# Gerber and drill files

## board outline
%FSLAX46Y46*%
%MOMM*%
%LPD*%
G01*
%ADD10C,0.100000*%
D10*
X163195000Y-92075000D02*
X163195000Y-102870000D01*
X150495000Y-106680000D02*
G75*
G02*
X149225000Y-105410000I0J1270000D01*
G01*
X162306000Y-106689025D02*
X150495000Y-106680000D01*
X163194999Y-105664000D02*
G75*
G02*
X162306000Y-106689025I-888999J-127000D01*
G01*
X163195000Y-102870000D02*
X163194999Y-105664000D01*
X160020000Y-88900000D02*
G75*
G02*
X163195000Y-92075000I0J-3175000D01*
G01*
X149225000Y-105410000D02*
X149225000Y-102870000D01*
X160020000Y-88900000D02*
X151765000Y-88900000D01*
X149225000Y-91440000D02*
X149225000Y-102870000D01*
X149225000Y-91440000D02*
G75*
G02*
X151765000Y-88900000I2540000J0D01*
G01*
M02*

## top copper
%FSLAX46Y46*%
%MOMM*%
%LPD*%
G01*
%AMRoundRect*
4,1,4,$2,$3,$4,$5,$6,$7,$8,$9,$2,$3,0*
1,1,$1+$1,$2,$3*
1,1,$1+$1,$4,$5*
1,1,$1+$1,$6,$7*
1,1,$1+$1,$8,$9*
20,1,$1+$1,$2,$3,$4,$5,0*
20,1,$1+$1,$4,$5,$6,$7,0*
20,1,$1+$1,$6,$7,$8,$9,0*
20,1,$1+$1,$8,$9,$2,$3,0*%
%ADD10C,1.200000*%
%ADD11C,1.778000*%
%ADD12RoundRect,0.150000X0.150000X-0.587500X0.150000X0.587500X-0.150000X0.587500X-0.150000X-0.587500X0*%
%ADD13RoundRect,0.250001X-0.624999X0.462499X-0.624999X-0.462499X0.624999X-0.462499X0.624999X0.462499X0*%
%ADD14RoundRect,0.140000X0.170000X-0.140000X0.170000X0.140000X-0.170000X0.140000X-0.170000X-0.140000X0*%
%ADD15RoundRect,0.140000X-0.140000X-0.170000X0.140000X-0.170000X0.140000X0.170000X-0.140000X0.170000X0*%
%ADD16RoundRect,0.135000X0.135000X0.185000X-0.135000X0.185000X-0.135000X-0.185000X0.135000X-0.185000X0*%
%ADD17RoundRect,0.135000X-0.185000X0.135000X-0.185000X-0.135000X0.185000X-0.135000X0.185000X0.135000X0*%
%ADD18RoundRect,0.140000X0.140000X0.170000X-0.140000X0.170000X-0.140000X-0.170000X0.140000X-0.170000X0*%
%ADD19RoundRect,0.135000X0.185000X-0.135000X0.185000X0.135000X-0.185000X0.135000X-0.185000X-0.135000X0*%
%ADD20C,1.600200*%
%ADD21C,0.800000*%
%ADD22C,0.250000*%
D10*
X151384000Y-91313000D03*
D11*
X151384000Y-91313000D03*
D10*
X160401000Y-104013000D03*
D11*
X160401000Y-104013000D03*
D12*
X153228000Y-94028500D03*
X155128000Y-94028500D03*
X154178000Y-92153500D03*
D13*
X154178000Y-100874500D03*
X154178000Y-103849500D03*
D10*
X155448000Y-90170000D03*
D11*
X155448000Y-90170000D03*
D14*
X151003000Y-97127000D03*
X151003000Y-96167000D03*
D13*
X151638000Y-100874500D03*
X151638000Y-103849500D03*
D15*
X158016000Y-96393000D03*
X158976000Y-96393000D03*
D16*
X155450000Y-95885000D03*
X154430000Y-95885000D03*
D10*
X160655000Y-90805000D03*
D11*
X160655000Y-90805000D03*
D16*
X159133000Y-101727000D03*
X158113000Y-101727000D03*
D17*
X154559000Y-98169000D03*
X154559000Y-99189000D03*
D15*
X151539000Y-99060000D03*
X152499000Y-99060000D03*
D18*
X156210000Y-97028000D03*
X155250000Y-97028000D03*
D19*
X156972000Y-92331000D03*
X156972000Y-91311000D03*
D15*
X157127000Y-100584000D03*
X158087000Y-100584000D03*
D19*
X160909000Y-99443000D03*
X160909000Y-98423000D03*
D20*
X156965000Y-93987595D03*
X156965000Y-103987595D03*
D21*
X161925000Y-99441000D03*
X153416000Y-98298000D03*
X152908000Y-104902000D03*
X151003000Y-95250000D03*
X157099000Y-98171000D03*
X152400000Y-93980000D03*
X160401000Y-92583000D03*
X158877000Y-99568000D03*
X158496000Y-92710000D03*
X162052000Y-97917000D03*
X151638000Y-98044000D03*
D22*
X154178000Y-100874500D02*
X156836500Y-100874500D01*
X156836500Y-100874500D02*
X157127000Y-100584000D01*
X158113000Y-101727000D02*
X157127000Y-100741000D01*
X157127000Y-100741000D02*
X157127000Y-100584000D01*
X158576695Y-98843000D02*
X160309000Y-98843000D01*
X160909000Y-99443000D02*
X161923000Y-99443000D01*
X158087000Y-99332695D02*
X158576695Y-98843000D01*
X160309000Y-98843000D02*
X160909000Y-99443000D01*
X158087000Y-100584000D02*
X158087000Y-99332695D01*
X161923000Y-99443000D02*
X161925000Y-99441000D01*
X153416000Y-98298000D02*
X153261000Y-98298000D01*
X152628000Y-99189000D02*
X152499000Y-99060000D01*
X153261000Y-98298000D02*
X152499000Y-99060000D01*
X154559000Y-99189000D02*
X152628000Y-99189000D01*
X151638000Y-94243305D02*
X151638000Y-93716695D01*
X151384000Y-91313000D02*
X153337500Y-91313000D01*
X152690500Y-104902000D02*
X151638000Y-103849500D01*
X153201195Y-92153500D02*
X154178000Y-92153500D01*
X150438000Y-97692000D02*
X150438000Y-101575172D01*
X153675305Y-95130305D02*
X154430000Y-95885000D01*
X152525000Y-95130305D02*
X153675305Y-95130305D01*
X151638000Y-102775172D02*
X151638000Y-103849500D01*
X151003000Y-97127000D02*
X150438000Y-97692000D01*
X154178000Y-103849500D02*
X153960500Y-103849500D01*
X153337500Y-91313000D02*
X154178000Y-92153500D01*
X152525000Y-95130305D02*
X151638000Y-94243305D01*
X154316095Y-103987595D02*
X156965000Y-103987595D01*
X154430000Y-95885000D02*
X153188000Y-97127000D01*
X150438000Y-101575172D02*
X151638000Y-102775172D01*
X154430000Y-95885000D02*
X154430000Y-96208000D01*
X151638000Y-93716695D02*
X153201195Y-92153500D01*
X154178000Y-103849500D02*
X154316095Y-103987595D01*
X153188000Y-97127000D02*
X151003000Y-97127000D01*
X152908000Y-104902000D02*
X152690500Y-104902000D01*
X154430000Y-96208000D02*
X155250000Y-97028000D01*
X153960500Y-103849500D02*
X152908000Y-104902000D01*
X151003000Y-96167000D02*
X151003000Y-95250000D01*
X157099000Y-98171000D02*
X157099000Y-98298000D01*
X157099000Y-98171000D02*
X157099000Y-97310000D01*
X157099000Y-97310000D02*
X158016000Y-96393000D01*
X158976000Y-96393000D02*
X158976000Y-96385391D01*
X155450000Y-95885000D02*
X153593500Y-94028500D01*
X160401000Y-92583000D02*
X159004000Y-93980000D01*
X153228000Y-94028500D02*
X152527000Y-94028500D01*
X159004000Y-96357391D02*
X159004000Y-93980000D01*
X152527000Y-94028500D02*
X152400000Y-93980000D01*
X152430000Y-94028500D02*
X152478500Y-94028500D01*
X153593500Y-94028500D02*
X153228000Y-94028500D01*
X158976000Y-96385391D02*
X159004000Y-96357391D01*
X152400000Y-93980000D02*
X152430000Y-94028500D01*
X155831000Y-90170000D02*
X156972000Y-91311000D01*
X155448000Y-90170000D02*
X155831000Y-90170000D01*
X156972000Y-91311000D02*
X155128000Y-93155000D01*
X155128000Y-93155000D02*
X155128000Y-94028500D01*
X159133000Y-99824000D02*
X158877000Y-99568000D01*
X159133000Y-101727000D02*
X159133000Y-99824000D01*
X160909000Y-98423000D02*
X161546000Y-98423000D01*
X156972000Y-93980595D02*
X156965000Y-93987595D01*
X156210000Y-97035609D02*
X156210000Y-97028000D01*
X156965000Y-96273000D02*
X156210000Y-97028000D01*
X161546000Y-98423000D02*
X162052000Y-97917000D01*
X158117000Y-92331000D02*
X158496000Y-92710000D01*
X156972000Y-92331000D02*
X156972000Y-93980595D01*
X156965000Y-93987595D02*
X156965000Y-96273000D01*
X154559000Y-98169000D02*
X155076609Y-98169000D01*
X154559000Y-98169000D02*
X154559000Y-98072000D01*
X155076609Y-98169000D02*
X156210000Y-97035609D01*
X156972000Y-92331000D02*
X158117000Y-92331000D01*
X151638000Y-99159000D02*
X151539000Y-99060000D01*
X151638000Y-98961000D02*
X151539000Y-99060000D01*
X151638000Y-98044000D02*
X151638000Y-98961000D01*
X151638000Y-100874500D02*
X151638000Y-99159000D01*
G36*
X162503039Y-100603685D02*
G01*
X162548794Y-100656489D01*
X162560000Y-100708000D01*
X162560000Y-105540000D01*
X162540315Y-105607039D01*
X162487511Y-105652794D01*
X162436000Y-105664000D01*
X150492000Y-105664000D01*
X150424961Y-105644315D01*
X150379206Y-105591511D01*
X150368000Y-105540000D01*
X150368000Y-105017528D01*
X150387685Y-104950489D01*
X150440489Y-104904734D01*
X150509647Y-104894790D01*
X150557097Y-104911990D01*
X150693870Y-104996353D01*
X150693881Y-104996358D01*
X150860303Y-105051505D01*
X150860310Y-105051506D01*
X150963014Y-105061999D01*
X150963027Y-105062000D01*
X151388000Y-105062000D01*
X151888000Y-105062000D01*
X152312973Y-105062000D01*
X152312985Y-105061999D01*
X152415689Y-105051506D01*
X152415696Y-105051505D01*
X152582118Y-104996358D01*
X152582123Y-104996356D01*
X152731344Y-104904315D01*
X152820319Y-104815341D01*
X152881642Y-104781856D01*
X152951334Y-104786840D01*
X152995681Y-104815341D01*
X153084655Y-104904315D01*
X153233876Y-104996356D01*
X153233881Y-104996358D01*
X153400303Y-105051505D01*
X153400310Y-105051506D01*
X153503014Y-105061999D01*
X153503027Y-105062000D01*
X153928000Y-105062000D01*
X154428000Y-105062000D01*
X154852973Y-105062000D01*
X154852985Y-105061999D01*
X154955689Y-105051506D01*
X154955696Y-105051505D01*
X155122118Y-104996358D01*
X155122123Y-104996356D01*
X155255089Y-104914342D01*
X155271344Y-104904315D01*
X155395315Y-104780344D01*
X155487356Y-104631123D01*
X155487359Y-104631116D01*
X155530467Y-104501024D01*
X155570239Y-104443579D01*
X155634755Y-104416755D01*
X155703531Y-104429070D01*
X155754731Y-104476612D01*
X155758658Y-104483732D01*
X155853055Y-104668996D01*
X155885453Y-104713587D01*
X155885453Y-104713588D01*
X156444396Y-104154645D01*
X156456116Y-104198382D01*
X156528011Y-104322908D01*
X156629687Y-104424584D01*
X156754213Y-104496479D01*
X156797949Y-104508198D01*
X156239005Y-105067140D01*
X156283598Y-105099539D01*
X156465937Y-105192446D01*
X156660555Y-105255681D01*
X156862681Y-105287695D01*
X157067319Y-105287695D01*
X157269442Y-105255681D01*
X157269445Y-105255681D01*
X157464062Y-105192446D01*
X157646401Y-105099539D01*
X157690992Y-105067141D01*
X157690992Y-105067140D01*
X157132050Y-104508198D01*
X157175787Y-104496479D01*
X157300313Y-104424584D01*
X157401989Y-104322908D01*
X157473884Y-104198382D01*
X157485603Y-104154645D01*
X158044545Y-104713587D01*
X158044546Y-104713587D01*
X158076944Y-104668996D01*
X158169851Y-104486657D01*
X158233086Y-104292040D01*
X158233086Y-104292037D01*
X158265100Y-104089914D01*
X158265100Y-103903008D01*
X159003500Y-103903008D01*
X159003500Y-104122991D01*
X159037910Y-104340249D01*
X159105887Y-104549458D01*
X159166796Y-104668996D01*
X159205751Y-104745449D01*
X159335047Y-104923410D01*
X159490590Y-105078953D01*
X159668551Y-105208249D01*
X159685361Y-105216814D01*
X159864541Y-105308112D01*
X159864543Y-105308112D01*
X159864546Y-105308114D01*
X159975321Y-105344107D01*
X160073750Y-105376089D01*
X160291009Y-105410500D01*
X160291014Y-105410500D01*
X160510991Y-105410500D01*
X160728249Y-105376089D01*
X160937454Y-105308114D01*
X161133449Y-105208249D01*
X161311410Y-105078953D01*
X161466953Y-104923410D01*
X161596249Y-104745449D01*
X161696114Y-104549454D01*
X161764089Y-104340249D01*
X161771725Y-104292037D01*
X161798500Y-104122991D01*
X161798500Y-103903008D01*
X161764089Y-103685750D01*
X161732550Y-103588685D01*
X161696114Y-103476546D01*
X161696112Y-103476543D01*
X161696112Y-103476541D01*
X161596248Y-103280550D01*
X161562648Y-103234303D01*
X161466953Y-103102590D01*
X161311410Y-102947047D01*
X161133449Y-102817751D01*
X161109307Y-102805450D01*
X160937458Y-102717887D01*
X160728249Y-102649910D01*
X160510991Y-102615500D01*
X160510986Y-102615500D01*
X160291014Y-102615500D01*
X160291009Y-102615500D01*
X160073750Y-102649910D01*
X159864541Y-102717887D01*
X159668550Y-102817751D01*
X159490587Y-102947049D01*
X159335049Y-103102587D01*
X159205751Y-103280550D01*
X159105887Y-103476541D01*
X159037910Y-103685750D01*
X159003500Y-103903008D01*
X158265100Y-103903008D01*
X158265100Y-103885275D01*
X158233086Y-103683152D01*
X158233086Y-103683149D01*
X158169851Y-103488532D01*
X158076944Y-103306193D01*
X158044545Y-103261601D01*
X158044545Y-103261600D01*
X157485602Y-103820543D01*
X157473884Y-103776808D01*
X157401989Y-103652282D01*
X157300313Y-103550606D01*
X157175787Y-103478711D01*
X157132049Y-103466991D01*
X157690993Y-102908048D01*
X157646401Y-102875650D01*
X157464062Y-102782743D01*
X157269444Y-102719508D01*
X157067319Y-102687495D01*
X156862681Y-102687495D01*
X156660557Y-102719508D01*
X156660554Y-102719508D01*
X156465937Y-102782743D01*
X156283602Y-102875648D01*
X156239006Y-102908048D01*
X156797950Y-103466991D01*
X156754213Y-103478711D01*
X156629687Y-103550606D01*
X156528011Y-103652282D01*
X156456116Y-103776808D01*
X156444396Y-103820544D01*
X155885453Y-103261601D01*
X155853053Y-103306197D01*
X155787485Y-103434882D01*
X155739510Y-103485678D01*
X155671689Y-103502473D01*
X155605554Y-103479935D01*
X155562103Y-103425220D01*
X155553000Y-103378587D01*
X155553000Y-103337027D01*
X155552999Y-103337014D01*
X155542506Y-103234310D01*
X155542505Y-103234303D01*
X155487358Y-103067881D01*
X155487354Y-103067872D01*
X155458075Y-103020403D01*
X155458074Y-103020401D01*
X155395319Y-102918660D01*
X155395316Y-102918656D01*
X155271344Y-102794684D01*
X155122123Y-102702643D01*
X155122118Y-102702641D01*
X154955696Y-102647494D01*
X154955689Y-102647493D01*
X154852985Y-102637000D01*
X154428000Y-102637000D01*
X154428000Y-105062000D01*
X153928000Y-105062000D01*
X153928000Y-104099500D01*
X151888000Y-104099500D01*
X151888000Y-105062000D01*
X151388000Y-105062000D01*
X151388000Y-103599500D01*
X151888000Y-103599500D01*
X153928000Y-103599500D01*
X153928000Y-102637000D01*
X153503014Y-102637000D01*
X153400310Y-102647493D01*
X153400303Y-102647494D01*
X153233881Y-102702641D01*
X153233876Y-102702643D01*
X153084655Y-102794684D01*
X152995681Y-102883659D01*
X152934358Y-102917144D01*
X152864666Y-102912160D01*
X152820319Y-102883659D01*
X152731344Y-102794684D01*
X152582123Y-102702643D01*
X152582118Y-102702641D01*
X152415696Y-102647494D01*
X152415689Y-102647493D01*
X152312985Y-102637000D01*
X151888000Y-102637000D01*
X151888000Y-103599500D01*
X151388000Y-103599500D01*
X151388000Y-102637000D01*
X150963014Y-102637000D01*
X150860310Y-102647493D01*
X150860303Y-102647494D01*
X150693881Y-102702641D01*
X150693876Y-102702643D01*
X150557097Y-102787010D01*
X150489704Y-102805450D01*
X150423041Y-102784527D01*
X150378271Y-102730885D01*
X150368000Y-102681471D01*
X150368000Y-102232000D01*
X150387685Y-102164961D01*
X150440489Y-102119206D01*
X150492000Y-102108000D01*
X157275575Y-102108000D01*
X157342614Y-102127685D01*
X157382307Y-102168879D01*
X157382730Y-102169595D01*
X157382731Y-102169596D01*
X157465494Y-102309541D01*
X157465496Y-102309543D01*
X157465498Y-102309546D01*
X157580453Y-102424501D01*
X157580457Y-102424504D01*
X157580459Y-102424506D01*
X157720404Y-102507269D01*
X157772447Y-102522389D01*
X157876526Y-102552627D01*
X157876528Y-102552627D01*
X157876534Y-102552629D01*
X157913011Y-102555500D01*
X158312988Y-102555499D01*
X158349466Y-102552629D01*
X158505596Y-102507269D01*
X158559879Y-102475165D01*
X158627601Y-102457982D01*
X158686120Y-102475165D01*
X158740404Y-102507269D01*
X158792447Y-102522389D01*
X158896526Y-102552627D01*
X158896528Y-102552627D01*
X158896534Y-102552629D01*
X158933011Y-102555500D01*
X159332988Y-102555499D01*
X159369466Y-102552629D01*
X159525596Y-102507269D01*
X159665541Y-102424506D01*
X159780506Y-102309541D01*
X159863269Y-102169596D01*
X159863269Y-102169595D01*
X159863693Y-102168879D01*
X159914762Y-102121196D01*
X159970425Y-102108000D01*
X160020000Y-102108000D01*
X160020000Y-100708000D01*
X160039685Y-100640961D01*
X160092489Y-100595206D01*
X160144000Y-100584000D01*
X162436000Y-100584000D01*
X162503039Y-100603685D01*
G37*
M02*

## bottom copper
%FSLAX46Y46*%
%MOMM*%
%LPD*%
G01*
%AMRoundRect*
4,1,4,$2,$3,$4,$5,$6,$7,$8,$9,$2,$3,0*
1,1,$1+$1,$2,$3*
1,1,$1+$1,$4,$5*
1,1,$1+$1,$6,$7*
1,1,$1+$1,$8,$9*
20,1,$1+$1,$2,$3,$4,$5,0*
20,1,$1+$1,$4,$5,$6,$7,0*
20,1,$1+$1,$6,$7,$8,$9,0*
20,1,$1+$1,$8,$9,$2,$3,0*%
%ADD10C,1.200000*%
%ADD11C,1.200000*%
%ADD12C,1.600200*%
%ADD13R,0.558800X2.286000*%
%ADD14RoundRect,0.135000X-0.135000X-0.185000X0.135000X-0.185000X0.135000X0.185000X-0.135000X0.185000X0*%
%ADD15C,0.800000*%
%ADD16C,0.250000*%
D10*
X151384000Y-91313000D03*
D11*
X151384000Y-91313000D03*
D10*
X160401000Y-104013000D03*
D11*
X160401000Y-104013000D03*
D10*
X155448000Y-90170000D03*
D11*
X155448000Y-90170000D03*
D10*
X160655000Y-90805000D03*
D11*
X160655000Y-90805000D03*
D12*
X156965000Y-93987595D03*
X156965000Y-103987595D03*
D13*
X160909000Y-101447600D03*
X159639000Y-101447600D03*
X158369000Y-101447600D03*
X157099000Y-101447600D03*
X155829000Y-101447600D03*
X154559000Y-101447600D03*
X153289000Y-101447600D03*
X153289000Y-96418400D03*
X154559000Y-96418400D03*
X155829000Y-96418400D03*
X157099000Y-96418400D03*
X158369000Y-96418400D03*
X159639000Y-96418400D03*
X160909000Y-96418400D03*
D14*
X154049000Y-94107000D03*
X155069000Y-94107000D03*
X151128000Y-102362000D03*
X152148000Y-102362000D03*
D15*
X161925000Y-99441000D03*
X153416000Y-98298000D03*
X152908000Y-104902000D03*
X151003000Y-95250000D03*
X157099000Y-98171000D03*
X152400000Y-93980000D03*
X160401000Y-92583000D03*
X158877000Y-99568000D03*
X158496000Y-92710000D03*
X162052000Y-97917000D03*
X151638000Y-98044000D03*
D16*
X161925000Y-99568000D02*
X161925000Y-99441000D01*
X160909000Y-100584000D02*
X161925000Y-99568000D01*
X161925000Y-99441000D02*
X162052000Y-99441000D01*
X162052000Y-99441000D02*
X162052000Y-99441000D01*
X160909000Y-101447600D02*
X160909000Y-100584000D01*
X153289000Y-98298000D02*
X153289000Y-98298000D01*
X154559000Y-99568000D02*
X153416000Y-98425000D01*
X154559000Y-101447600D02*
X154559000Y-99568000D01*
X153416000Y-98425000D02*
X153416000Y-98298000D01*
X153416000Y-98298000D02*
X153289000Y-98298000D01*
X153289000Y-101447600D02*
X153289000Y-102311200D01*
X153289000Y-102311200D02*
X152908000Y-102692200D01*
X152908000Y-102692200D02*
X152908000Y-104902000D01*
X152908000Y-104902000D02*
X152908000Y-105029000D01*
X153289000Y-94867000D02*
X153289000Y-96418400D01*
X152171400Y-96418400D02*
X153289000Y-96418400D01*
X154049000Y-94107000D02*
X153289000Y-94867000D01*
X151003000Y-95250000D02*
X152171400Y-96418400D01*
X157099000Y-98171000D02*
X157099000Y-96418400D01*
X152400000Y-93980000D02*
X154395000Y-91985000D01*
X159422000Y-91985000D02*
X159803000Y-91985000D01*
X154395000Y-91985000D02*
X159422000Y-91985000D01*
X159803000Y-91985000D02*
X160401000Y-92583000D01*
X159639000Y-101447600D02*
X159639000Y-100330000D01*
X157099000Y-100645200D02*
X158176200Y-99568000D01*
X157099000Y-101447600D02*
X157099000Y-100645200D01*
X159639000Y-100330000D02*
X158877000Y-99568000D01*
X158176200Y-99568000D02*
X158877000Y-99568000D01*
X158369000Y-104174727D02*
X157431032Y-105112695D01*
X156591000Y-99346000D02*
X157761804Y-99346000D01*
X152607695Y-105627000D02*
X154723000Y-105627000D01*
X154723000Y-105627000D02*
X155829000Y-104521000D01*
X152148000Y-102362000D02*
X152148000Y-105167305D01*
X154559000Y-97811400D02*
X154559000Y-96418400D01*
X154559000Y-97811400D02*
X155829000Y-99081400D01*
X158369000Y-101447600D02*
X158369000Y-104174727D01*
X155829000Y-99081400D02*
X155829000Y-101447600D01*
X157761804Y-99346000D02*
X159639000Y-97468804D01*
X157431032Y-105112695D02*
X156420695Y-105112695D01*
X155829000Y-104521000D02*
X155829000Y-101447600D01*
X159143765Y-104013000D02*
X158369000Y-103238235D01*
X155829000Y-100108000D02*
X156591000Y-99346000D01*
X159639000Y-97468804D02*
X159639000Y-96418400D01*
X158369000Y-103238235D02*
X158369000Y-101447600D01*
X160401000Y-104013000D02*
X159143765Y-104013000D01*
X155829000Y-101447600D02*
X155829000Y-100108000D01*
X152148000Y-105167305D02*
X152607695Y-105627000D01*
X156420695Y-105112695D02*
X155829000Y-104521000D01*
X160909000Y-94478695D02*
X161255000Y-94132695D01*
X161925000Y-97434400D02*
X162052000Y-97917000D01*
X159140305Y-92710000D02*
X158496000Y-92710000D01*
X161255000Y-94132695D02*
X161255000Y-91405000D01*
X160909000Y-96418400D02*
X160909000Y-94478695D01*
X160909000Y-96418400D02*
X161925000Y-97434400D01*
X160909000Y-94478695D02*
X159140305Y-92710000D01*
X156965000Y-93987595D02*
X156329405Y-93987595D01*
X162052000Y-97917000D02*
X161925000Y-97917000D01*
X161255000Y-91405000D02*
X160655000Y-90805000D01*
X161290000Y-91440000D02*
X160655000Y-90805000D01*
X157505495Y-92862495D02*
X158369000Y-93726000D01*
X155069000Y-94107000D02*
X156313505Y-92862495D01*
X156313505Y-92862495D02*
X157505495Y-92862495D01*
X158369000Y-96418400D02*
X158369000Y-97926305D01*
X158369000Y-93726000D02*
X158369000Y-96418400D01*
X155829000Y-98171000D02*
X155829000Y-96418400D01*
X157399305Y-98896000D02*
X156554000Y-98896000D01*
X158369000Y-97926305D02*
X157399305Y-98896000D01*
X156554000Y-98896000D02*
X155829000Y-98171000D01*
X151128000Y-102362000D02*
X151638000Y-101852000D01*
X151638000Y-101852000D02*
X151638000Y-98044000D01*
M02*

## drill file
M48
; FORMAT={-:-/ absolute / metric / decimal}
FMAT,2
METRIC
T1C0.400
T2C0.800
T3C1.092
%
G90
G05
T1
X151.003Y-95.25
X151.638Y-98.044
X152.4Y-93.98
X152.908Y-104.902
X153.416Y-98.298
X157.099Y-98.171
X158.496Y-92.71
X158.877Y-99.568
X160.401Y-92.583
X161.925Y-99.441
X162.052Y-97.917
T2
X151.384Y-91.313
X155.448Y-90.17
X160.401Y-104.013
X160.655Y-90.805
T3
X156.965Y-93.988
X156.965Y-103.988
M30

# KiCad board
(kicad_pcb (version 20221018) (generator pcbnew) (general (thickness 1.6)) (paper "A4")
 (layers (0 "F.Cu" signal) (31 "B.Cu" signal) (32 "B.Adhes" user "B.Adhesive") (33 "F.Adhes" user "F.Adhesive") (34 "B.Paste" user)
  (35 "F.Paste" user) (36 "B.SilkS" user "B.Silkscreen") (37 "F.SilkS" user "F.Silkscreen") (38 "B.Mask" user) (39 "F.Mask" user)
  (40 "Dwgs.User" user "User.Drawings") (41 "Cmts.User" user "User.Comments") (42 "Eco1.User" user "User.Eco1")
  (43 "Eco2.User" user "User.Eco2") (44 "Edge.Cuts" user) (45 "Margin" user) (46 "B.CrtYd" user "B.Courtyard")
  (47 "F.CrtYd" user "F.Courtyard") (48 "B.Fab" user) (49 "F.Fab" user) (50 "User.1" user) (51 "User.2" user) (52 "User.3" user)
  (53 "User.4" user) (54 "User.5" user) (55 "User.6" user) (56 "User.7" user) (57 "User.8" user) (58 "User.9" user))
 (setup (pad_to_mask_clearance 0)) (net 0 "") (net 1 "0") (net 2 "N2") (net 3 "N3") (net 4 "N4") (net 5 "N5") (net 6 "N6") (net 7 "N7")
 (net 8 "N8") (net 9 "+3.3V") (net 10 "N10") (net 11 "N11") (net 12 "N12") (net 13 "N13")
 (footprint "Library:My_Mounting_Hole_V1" (layer "F.Cu") (at 151.384 91.313)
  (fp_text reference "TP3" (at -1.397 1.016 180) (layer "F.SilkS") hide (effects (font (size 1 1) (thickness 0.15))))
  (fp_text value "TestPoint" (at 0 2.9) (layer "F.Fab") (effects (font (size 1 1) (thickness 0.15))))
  (pad "1" thru_hole circle (at 0 0) (size 1.2 1.2) (drill 0.8) (layers "*.Cu" "*.Mask") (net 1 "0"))
  (pad "1" connect circle (at 0 0) (size 1.2 1.2) (layers "B.Cu" "B.Mask") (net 1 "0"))
  (pad "1" connect circle (at 0 0) (size 1.778 1.778) (layers "F.Cu" "F.Mask") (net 1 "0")))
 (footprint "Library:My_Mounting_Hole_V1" (layer "F.Cu") (at 160.401 104.013)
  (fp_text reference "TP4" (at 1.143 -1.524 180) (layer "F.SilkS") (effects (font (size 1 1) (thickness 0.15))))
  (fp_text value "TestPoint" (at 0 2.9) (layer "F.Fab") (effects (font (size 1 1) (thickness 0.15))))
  (pad "1" thru_hole circle (at 0 0) (size 1.2 1.2) (drill 0.8) (layers "*.Cu" "*.Mask") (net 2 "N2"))
  (pad "1" connect circle (at 0 0) (size 1.2 1.2) (layers "B.Cu" "B.Mask") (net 2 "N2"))
  (pad "1" connect circle (at 0 0) (size 1.778 1.778) (layers "F.Cu" "F.Mask") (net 2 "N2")))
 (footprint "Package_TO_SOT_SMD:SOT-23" (layer "F.Cu") (at 154.178 93.091 90)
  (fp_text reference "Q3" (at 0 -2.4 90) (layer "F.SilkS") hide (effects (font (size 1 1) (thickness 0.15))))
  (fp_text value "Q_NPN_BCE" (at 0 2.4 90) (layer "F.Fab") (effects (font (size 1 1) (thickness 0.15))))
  (pad "1" smd roundrect (at -0.9375 -0.95 90) (size 1.475 0.6) (layers "F.Cu" "F.Paste" "F.Mask") (roundrect_rratio 0.25) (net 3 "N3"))
  (pad "2" smd roundrect (at -0.9375 0.95 90) (size 1.475 0.6) (layers "F.Cu" "F.Paste" "F.Mask") (roundrect_rratio 0.25) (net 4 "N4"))
  (pad "3" smd roundrect (at 0.9375 0 90) (size 1.475 0.6) (layers "F.Cu" "F.Paste" "F.Mask") (roundrect_rratio 0.25) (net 1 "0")))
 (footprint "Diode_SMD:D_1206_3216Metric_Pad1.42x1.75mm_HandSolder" (layer "F.Cu") (at 154.178 102.362 -90)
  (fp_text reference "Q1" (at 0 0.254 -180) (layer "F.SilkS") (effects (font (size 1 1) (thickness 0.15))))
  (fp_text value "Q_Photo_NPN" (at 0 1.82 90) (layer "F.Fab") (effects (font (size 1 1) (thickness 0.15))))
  (pad "1" smd roundrect (at -1.4875 0 270) (size 1.425 1.75) (layers "F.Cu" "F.Paste" "F.Mask") (roundrect_rratio 0.1754392982)
   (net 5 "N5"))
  (pad "2" smd roundrect (at 1.4875 0 270) (size 1.425 1.75) (layers "F.Cu" "F.Paste" "F.Mask") (roundrect_rratio 0.1754392982) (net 1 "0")))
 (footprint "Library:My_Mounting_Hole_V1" (layer "F.Cu") (at 155.448 90.17)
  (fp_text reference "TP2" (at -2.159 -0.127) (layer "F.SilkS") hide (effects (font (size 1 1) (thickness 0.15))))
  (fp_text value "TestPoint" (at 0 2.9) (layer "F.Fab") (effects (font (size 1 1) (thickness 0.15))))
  (pad "1" thru_hole circle (at 0 0) (size 1.2 1.2) (drill 0.8) (layers "*.Cu" "*.Mask") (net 4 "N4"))
  (pad "1" connect circle (at 0 0) (size 1.2 1.2) (layers "B.Cu" "B.Mask") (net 4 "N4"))
  (pad "1" connect circle (at 0 0) (size 1.778 1.778) (layers "F.Cu" "F.Mask") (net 4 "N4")))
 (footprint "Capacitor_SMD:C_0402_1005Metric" (layer "F.Cu") (at 151.003 96.647 90)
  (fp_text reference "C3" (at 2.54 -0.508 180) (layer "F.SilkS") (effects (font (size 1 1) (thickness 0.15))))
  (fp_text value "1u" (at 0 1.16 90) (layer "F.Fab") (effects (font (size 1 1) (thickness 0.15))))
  (pad "1" smd roundrect (at -0.48 0 90) (size 0.56 0.62) (layers "F.Cu" "F.Paste" "F.Mask") (roundrect_rratio 0.25) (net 1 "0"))
  (pad "2" smd roundrect (at 0.48 0 90) (size 0.56 0.62) (layers "F.Cu" "F.Paste" "F.Mask") (roundrect_rratio 0.25) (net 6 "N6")))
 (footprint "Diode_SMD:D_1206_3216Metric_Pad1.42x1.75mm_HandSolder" (layer "F.Cu") (at 151.638 102.362 -90)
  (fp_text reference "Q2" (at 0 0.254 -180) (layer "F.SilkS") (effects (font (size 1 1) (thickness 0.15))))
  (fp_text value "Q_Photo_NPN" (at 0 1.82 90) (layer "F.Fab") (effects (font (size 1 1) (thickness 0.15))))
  (pad "1" smd roundrect (at -1.4875 0 270) (size 1.425 1.75) (layers "F.Cu" "F.Paste" "F.Mask") (roundrect_rratio 0.1754392982)
   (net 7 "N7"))
  (pad "2" smd roundrect (at 1.4875 0 270) (size 1.425 1.75) (layers "F.Cu" "F.Paste" "F.Mask") (roundrect_rratio 0.1754392982) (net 1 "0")))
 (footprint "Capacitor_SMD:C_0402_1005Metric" (layer "F.Cu") (at 158.496 96.393)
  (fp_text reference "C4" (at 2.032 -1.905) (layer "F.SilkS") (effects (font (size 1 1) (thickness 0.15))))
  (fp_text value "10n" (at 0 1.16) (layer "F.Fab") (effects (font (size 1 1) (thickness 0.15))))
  (pad "1" smd roundrect (at -0.48 0) (size 0.56 0.62) (layers "F.Cu" "F.Paste" "F.Mask") (roundrect_rratio 0.25) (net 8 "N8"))
  (pad "2" smd roundrect (at 0.48 0) (size 0.56 0.62) (layers "F.Cu" "F.Paste" "F.Mask") (roundrect_rratio 0.25) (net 3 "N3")))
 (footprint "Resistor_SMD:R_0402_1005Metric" (layer "F.Cu") (at 154.94 95.885 180)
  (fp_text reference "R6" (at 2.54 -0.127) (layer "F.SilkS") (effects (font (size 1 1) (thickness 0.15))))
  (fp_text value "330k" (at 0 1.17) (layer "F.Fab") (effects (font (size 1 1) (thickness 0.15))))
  (pad "1" smd roundrect (at -0.51 0 180) (size 0.54 0.64) (layers "F.Cu" "F.Paste" "F.Mask") (roundrect_rratio 0.25) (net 3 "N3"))
  (pad "2" smd roundrect (at 0.51 0 180) (size 0.54 0.64) (layers "F.Cu" "F.Paste" "F.Mask") (roundrect_rratio 0.25) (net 1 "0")))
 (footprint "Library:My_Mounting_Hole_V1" (layer "F.Cu") (at 160.655 90.805)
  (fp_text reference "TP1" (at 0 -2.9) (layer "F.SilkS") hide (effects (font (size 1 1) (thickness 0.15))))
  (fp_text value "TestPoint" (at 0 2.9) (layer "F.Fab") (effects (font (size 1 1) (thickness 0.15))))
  (pad "1" thru_hole circle (at 0 0) (size 1.2 1.2) (drill 0.8) (layers "*.Cu" "*.Mask") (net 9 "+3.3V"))
  (pad "1" connect circle (at 0 0) (size 1.2 1.2) (layers "B.Cu" "B.Mask") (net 9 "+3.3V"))
  (pad "1" connect circle (at 0 0) (size 1.778 1.778) (layers "F.Cu" "F.Mask") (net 9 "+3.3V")))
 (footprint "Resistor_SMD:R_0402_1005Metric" (layer "F.Cu") (at 158.623 101.727 180)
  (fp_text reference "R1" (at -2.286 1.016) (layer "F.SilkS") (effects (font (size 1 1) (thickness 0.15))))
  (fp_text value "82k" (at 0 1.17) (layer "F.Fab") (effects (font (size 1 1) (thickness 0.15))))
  (pad "1" smd roundrect (at -0.51 0 180) (size 0.54 0.64) (layers "F.Cu" "F.Paste" "F.Mask") (roundrect_rratio 0.25) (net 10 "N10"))
  (pad "2" smd roundrect (at 0.51 0 180) (size 0.54 0.64) (layers "F.Cu" "F.Paste" "F.Mask") (roundrect_rratio 0.25) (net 5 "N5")))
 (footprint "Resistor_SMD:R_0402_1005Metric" (layer "F.Cu") (at 154.559 98.679 -90)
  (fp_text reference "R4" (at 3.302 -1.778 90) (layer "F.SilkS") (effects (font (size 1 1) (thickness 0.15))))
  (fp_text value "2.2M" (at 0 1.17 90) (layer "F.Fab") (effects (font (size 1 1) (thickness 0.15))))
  (pad "1" smd roundrect (at -0.51 0 270) (size 0.54 0.64) (layers "F.Cu" "F.Paste" "F.Mask") (roundrect_rratio 0.25) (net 9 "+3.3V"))
  (pad "2" smd roundrect (at 0.51 0 270) (size 0.54 0.64) (layers "F.Cu" "F.Paste" "F.Mask") (roundrect_rratio 0.25) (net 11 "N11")))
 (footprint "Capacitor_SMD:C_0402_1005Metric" (layer "F.Cu") (at 152.019 99.06)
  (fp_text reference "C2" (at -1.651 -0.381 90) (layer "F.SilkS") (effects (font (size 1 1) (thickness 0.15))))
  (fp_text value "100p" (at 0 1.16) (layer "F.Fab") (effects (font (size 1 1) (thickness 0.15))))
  (pad "1" smd roundrect (at -0.48 0) (size 0.56 0.62) (layers "F.Cu" "F.Paste" "F.Mask") (roundrect_rratio 0.25) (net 7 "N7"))
  (pad "2" smd roundrect (at 0.48 0) (size 0.56 0.62) (layers "F.Cu" "F.Paste" "F.Mask") (roundrect_rratio 0.25) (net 11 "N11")))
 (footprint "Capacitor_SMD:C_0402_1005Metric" (layer "F.Cu") (at 155.73 97.028 180)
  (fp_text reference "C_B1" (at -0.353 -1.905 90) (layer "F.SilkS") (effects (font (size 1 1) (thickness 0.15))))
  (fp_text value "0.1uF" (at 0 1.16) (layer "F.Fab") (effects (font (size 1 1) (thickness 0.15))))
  (pad "1" smd roundrect (at -0.48 0 180) (size 0.56 0.62) (layers "F.Cu" "F.Paste" "F.Mask") (roundrect_rratio 0.25) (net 9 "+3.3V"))
  (pad "2" smd roundrect (at 0.48 0 180) (size 0.56 0.62) (layers "F.Cu" "F.Paste" "F.Mask") (roundrect_rratio 0.25) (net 1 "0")))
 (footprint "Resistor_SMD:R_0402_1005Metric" (layer "F.Cu") (at 156.972 91.821 90)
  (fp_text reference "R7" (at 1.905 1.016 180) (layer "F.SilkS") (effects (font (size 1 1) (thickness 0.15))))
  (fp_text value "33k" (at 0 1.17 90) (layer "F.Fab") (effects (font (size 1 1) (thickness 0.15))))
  (pad "1" smd roundrect (at -0.51 0 90) (size 0.54 0.64) (layers "F.Cu" "F.Paste" "F.Mask") (roundrect_rratio 0.25) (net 9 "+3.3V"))
  (pad "2" smd roundrect (at 0.51 0 90) (size 0.54 0.64) (layers "F.Cu" "F.Paste" "F.Mask") (roundrect_rratio 0.25) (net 4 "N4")))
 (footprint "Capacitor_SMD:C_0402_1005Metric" (layer "F.Cu") (at 157.607 100.584)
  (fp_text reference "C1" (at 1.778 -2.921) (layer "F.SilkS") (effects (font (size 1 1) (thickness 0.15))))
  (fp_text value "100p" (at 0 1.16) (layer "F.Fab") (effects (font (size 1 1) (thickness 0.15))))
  (pad "1" smd roundrect (at -0.48 0) (size 0.56 0.62) (layers "F.Cu" "F.Paste" "F.Mask") (roundrect_rratio 0.25) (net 5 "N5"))
  (pad "2" smd roundrect (at 0.48 0) (size 0.56 0.62) (layers "F.Cu" "F.Paste" "F.Mask") (roundrect_rratio 0.25) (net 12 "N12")))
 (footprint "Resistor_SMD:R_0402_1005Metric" (layer "F.Cu") (at 160.909 98.933 90)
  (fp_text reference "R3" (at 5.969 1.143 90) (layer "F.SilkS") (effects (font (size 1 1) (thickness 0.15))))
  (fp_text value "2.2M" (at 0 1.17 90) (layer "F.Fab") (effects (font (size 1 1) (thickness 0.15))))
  (pad "1" smd roundrect (at -0.51 0 90) (size 0.54 0.64) (layers "F.Cu" "F.Paste" "F.Mask") (roundrect_rratio 0.25) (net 12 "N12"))
  (pad "2" smd roundrect (at 0.51 0 90) (size 0.54 0.64) (layers "F.Cu" "F.Paste" "F.Mask") (roundrect_rratio 0.25) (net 9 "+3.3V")))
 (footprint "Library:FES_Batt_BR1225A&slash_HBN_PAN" (layer "B.Cu") (at 156.965 93.987595 180)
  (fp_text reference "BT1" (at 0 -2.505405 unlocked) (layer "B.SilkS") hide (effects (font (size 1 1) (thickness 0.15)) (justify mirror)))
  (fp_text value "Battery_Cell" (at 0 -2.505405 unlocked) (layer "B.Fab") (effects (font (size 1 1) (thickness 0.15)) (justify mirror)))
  (pad "1" thru_hole circle (at 0 0 180) (size 1.6002 1.6002) (drill 1.0922) (layers "*.Cu" "*.Mask") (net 9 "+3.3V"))
  (pad "2" thru_hole circle (at 0 -10 180) (size 1.6002 1.6002) (drill 1.0922) (layers "*.Cu" "*.Mask") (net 1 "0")))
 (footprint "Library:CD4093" (layer "B.Cu") (at 157.099 98.933 90)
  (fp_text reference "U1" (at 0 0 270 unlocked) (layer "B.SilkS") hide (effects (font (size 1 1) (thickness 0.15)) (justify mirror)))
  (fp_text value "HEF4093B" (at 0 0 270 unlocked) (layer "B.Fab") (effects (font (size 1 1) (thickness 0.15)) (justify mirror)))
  (pad "1" smd rect (at -2.5146 3.81 90) (size 2.286 0.5588) (layers "B.Cu" "B.Paste" "B.Mask") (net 12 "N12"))
  (pad "2" smd rect (at -2.5146 2.54 90) (size 2.286 0.5588) (layers "B.Cu" "B.Paste" "B.Mask") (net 10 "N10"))
  (pad "3" smd rect (at -2.5146 1.27 90) (size 2.286 0.5588) (layers "B.Cu" "B.Paste" "B.Mask") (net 2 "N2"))
  (pad "4" smd rect (at -2.5146 0 90) (size 2.286 0.5588) (layers "B.Cu" "B.Paste" "B.Mask") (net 10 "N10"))
  (pad "5" smd rect (at -2.5146 -1.27 90) (size 2.286 0.5588) (layers "B.Cu" "B.Paste" "B.Mask") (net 2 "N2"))
  (pad "6" smd rect (at -2.5146 -2.54 90) (size 2.286 0.5588) (layers "B.Cu" "B.Paste" "B.Mask") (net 11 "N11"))
  (pad "7" smd rect (at -2.5146 -3.81 90) (size 2.286 0.5588) (layers "B.Cu" "B.Paste" "B.Mask") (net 1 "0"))
  (pad "8" smd rect (at 2.5146 -3.81 90) (size 2.286 0.5588) (layers "B.Cu" "B.Paste" "B.Mask") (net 6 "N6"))
  (pad "9" smd rect (at 2.5146 -2.54 90) (size 2.286 0.5588) (layers "B.Cu" "B.Paste" "B.Mask") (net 2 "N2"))
  (pad "10" smd rect (at 2.5146 -1.27 90) (size 2.286 0.5588) (layers "B.Cu" "B.Paste" "B.Mask") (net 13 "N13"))
  (pad "11" smd rect (at 2.5146 0 90) (size 2.286 0.5588) (layers "B.Cu" "B.Paste" "B.Mask") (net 8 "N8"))
  (pad "12" smd rect (at 2.5146 1.27 90) (size 2.286 0.5588) (layers "B.Cu" "B.Paste" "B.Mask") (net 13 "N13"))
  (pad "13" smd rect (at 2.5146 2.54 90) (size 2.286 0.5588) (layers "B.Cu" "B.Paste" "B.Mask") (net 2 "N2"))
  (pad "14" smd rect (at 2.5146 3.81 90) (size 2.286 0.5588) (layers "B.Cu" "B.Paste" "B.Mask") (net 9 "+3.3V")))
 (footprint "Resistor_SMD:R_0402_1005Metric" (layer "B.Cu") (at 154.559 94.107)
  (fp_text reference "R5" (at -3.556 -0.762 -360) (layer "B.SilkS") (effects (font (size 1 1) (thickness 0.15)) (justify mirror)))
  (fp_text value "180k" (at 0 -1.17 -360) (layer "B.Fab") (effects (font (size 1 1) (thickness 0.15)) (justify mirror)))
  (pad "1" smd roundrect (at -0.51 0) (size 0.54 0.64) (layers "B.Cu" "B.Paste" "B.Mask") (roundrect_rratio 0.25) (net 6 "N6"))
  (pad "2" smd roundrect (at 0.51 0) (size 0.54 0.64) (layers "B.Cu" "B.Paste" "B.Mask") (roundrect_rratio 0.25) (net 13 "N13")))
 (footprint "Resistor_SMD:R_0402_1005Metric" (layer "B.Cu") (at 151.638 102.362)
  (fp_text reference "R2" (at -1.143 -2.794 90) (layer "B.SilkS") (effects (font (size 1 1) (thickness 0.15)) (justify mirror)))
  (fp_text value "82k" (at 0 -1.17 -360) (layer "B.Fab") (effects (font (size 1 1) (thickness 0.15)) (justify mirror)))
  (pad "1" smd roundrect (at -0.51 0) (size 0.54 0.64) (layers "B.Cu" "B.Paste" "B.Mask") (roundrect_rratio 0.25) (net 7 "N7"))
  (pad "2" smd roundrect (at 0.51 0) (size 0.54 0.64) (layers "B.Cu" "B.Paste" "B.Mask") (roundrect_rratio 0.25) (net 2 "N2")))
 (gr_line (start 163.195 92.075) (end 163.195 102.87) (stroke (width 0.1) (type default)) (layer "Edge.Cuts"))
 (gr_arc (start 150.495 106.68) (mid 149.596974 106.308026) (end 149.225 105.41) (stroke (width 0.1) (type default)) (layer "Edge.Cuts"))
 (gr_line (start 162.306 106.689025) (end 150.495 106.68) (stroke (width 0.1) (type default)) (layer "Edge.Cuts"))
 (gr_arc (start 163.194999 105.664) (mid 162.984416 106.379387) (end 162.306 106.689025) (stroke (width 0.1) (type default))
  (layer "Edge.Cuts"))
 (gr_line (start 163.195 102.87) (end 163.194999 105.664) (stroke (width 0.1) (type default)) (layer "Edge.Cuts"))
 (gr_arc (start 160.02 88.9) (mid 162.265064 89.829936) (end 163.195 92.075) (stroke (width 0.1) (type default)) (layer "Edge.Cuts"))
 (gr_line (start 149.225 105.41) (end 149.225 102.87) (stroke (width 0.1) (type default)) (layer "Edge.Cuts"))
 (gr_line (start 160.02 88.9) (end 151.765 88.9) (stroke (width 0.1) (type default)) (layer "Edge.Cuts"))
 (gr_line (start 149.225 91.44) (end 149.225 102.87) (stroke (width 0.1) (type default)) (layer "Edge.Cuts"))
 (gr_arc (start 149.225 91.44) (mid 149.968949 89.643949) (end 151.765 88.9) (stroke (width 0.1) (type default)) (layer "Edge.Cuts"))
 (segment (start 154.178 100.8745) (end 156.8365 100.8745) (width 0.25) (layer "F.Cu") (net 5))
 (segment (start 156.8365 100.8745) (end 157.127 100.584) (width 0.25) (layer "F.Cu") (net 5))
 (segment (start 158.113 101.727) (end 157.127 100.741) (width 0.25) (layer "F.Cu") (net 5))
 (segment (start 157.127 100.741) (end 157.127 100.584) (width 0.25) (layer "F.Cu") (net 5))
 (segment (start 158.576695 98.843) (end 160.309 98.843) (width 0.25) (layer "F.Cu") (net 12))
 (segment (start 160.909 99.443) (end 161.923 99.443) (width 0.25) (layer "F.Cu") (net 12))
 (segment (start 158.087 99.332695) (end 158.576695 98.843) (width 0.25) (layer "F.Cu") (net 12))
 (segment (start 160.309 98.843) (end 160.909 99.443) (width 0.25) (layer "F.Cu") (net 12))
 (segment (start 158.087 100.584) (end 158.087 99.332695) (width 0.25) (layer "F.Cu") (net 12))
 (segment (start 161.923 99.443) (end 161.925 99.441) (width 0.25) (layer "F.Cu") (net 12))
 (via (at 161.925 99.441) (size 0.8) (drill 0.4) (layers "F.Cu" "B.Cu") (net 12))
 (segment (start 161.925 99.568) (end 161.925 99.441) (width 0.25) (layer "B.Cu") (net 12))
 (segment (start 160.909 100.584) (end 161.925 99.568) (width 0.25) (layer "B.Cu") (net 12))
 (segment (start 161.925 99.441) (end 162.052 99.441) (width 0.25) (layer "B.Cu") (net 12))
 (segment (start 162.052 99.441) (end 162.052 99.441) (width 0.25) (layer "B.Cu") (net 12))
 (segment (start 160.909 101.4476) (end 160.909 100.584) (width 0.25) (layer "B.Cu") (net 12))
 (segment (start 153.416 98.298) (end 153.261 98.298) (width 0.25) (layer "F.Cu") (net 11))
 (segment (start 152.628 99.189) (end 152.499 99.06) (width 0.25) (layer "F.Cu") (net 11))
 (segment (start 153.261 98.298) (end 152.499 99.06) (width 0.25) (layer "F.Cu") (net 11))
 (segment (start 154.559 99.189) (end 152.628 99.189) (width 0.25) (layer "F.Cu") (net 11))
 (via (at 153.416 98.298) (size 0.8) (drill 0.4) (layers "F.Cu" "B.Cu") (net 11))
 (segment (start 153.289 98.298) (end 153.289 98.298) (width 0.25) (layer "B.Cu") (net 11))
 (segment (start 154.559 99.568) (end 153.416 98.425) (width 0.25) (layer "B.Cu") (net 11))
 (segment (start 154.559 101.4476) (end 154.559 99.568) (width 0.25) (layer "B.Cu") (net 11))
 (segment (start 153.416 98.425) (end 153.416 98.298) (width 0.25) (layer "B.Cu") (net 11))
 (segment (start 153.416 98.298) (end 153.289 98.298) (width 0.25) (layer "B.Cu") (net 11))
 (segment (start 151.638 94.243305) (end 151.638 93.716695) (width 0.25) (layer "F.Cu") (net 1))
 (segment (start 151.384 91.313) (end 153.3375 91.313) (width 0.25) (layer "F.Cu") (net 1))
 (segment (start 152.6905 104.902) (end 151.638 103.8495) (width 0.25) (layer "F.Cu") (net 1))
 (segment (start 153.201195 92.1535) (end 154.178 92.1535) (width 0.25) (layer "F.Cu") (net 1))
 (segment (start 150.438 97.692) (end 150.438 101.575172) (width 0.25) (layer "F.Cu") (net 1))
 (segment (start 153.675305 95.130305) (end 154.43 95.885) (width 0.25) (layer "F.Cu") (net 1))
 (segment (start 152.525 95.130305) (end 153.675305 95.130305) (width 0.25) (layer "F.Cu") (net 1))
 (segment (start 151.638 102.775172) (end 151.638 103.8495) (width 0.25) (layer "F.Cu") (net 1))
 (segment (start 151.003 97.127) (end 150.438 97.692) (width 0.25) (layer "F.Cu") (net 1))
 (segment (start 154.178 103.8495) (end 153.9605 103.8495) (width 0.25) (layer "F.Cu") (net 1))
 (segment (start 153.3375 91.313) (end 154.178 92.1535) (width 0.25) (layer "F.Cu") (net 1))
 (segment (start 152.525 95.130305) (end 151.638 94.243305) (width 0.25) (layer "F.Cu") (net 1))
 (segment (start 154.316095 103.987595) (end 156.965 103.987595) (width 0.25) (layer "F.Cu") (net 1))
 (segment (start 154.43 95.885) (end 153.188 97.127) (width 0.25) (layer "F.Cu") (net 1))
 (segment (start 150.438 101.575172) (end 151.638 102.775172) (width 0.25) (layer "F.Cu") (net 1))
 (segment (start 154.43 95.885) (end 154.43 96.208) (width 0.25) (layer "F.Cu") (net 1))
 (segment (start 151.638 93.716695) (end 153.201195 92.1535) (width 0.25) (layer "F.Cu") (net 1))
 (segment (start 154.178 103.8495) (end 154.316095 103.987595) (width 0.25) (layer "F.Cu") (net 1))
 (segment (start 153.188 97.127) (end 151.003 97.127) (width 0.25) (layer "F.Cu") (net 1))
 (segment (start 152.908 104.902) (end 152.6905 104.902) (width 0.25) (layer "F.Cu") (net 1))
 (segment (start 154.43 96.208) (end 155.25 97.028) (width 0.25) (layer "F.Cu") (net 1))
 (segment (start 153.9605 103.8495) (end 152.908 104.902) (width 0.25) (layer "F.Cu") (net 1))
 (via (at 152.908 104.902) (size 0.8) (drill 0.4) (layers "F.Cu" "B.Cu") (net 1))
 (segment (start 153.289 101.4476) (end 153.289 102.3112) (width 0.25) (layer "B.Cu") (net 1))
 (segment (start 153.289 102.3112) (end 152.908 102.6922) (width 0.25) (layer "B.Cu") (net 1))
 (segment (start 152.908 102.6922) (end 152.908 104.902) (width 0.25) (layer "B.Cu") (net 1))
 (segment (start 152.908 104.902) (end 152.908 105.029) (width 0.25) (layer "B.Cu") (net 1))
 (segment (start 151.003 96.167) (end 151.003 95.25) (width 0.25) (layer "F.Cu") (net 6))
 (via (at 151.003 95.25) (size 0.8) (drill 0.4) (layers "F.Cu" "B.Cu") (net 6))
 (segment (start 153.289 94.867) (end 153.289 96.4184) (width 0.25) (layer "B.Cu") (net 6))
 (segment (start 152.1714 96.4184) (end 153.289 96.4184) (width 0.25) (layer "B.Cu") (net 6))
 (segment (start 154.049 94.107) (end 153.289 94.867) (width 0.25) (layer "B.Cu") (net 6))
 (segment (start 151.003 95.25) (end 152.1714 96.4184) (width 0.25) (layer "B.Cu") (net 6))
 (segment (start 157.099 98.171) (end 157.099 98.298) (width 0.25) (layer "F.Cu") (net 8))
 (segment (start 157.099 98.171) (end 157.099 97.31) (width 0.25) (layer "F.Cu") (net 8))
 (segment (start 157.099 97.31) (end 158.016 96.393) (width 0.25) (layer "F.Cu") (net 8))
 (via (at 157.099 98.171) (size 0.8) (drill 0.4) (layers "F.Cu" "B.Cu") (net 8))
 (segment (start 157.099 98.171) (end 157.099 96.4184) (width 0.25) (layer "B.Cu") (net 8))
 (segment (start 158.976 96.393) (end 158.976 96.385391) (width 0.25) (layer "F.Cu") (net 3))
 (segment (start 155.45 95.885) (end 153.5935 94.0285) (width 0.25) (layer "F.Cu") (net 3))
 (segment (start 160.401 92.583) (end 159.004 93.98) (width 0.25) (layer "F.Cu") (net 3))
 (segment (start 153.228 94.0285) (end 152.527 94.0285) (width 0.25) (layer "F.Cu") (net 3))
 (segment (start 159.004 96.357391) (end 159.004 93.98) (width 0.25) (layer "F.Cu") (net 3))
 (segment (start 152.527 94.0285) (end 152.4 93.98) (width 0.25) (layer "F.Cu") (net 3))
 (segment (start 152.43 94.0285) (end 152.4785 94.0285) (width 0.25) (layer "F.Cu") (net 3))
 (segment (start 153.5935 94.0285) (end 153.228 94.0285) (width 0.25) (layer "F.Cu") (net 3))
 (segment (start 158.976 96.385391) (end 159.004 96.357391) (width 0.25) (layer "F.Cu") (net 3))
 (segment (start 152.4 93.98) (end 152.43 94.0285) (width 0.25) (layer "F.Cu") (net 3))
 (via (at 152.4 93.98) (size 0.8) (drill 0.4) (layers "F.Cu" "B.Cu") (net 3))
 (via (at 160.401 92.583) (size 0.8) (drill 0.4) (layers "F.Cu" "B.Cu") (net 3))
 (segment (start 152.4 93.98) (end 154.395 91.985) (width 0.25) (layer "B.Cu") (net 3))
 (segment (start 159.422 91.985) (end 159.803 91.985) (width 0.25) (layer "B.Cu") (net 3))
 (segment (start 154.395 91.985) (end 159.422 91.985) (width 0.25) (layer "B.Cu") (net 3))
 (segment (start 159.803 91.985) (end 160.401 92.583) (width 0.25) (layer "B.Cu") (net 3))
 (segment (start 155.831 90.17) (end 156.972 91.311) (width 0.25) (layer "F.Cu") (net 4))
 (segment (start 155.448 90.17) (end 155.831 90.17) (width 0.25) (layer "F.Cu") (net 4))
 (segment (start 156.972 91.311) (end 155.128 93.155) (width 0.25) (layer "F.Cu") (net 4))
 (segment (start 155.128 93.155) (end 155.128 94.0285) (width 0.25) (layer "F.Cu") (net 4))
 (segment (start 159.133 99.824) (end 158.877 99.568) (width 0.25) (layer "F.Cu") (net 10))
 (segment (start 159.133 101.727) (end 159.133 99.824) (width 0.25) (layer "F.Cu") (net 10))
 (via (at 158.877 99.568) (size 0.8) (drill 0.4) (layers "F.Cu" "B.Cu") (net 10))
 (segment (start 159.639 101.4476) (end 159.639 100.33) (width 0.25) (layer "B.Cu") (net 10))
 (segment (start 157.099 100.6452) (end 158.1762 99.568) (width 0.25) (layer "B.Cu") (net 10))
 (segment (start 157.099 101.4476) (end 157.099 100.6452) (width 0.25) (layer "B.Cu") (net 10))
 (segment (start 159.639 100.33) (end 158.877 99.568) (width 0.25) (layer "B.Cu") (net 10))
 (segment (start 158.1762 99.568) (end 158.877 99.568) (width 0.25) (layer "B.Cu") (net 10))
 (segment (start 158.369 104.174727) (end 157.431032 105.112695) (width 0.25) (layer "B.Cu") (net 2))
 (segment (start 156.591 99.346) (end 157.761804 99.346) (width 0.25) (layer "B.Cu") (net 2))
 (segment (start 152.607695 105.627) (end 154.723 105.627) (width 0.25) (layer "B.Cu") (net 2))
 (segment (start 154.723 105.627) (end 155.829 104.521) (width 0.25) (layer "B.Cu") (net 2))
 (segment (start 152.148 102.362) (end 152.148 105.167305) (width 0.25) (layer "B.Cu") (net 2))
 (segment (start 154.559 97.8114) (end 154.559 96.4184) (width 0.25) (layer "B.Cu") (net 2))
 (segment (start 154.559 97.8114) (end 155.829 99.0814) (width 0.25) (layer "B.Cu") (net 2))
 (segment (start 158.369 101.4476) (end 158.369 104.174727) (width 0.25) (layer "B.Cu") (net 2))
 (segment (start 155.829 99.0814) (end 155.829 101.4476) (width 0.25) (layer "B.Cu") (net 2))
 (segment (start 157.761804 99.346) (end 159.639 97.468804) (width 0.25) (layer "B.Cu") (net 2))
 (segment (start 157.431032 105.112695) (end 156.420695 105.112695) (width 0.25) (layer "B.Cu") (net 2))
 (segment (start 155.829 104.521) (end 155.829 101.4476) (width 0.25) (layer "B.Cu") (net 2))
 (segment (start 159.143765 104.013) (end 158.369 103.238235) (width 0.25) (layer "B.Cu") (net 2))
 (segment (start 155.829 100.108) (end 156.591 99.346) (width 0.25) (layer "B.Cu") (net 2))
 (segment (start 159.639 97.468804) (end 159.639 96.4184) (width 0.25) (layer "B.Cu") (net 2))
 (segment (start 158.369 103.238235) (end 158.369 101.4476) (width 0.25) (layer "B.Cu") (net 2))
 (segment (start 160.401 104.013) (end 159.143765 104.013) (width 0.25) (layer "B.Cu") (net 2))
 (segment (start 155.829 101.4476) (end 155.829 100.108) (width 0.25) (layer "B.Cu") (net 2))
 (segment (start 152.148 105.167305) (end 152.607695 105.627) (width 0.25) (layer "B.Cu") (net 2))
 (segment (start 156.420695 105.112695) (end 155.829 104.521) (width 0.25) (layer "B.Cu") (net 2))
 (segment (start 160.909 98.423) (end 161.546 98.423) (width 0.25) (layer "F.Cu") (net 9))
 (segment (start 156.972 93.980595) (end 156.965 93.987595) (width 0.25) (layer "F.Cu") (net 9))
 (segment (start 156.21 97.035609) (end 156.21 97.028) (width 0.25) (layer "F.Cu") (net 9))
 (segment (start 156.965 96.273) (end 156.21 97.028) (width 0.25) (layer "F.Cu") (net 9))
 (segment (start 161.546 98.423) (end 162.052 97.917) (width 0.25) (layer "F.Cu") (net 9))
 (segment (start 158.117 92.331) (end 158.496 92.71) (width 0.25) (layer "F.Cu") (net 9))
 (segment (start 156.972 92.331) (end 156.972 93.980595) (width 0.25) (layer "F.Cu") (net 9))
 (segment (start 156.965 93.987595) (end 156.965 96.273) (width 0.25) (layer "F.Cu") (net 9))
 (segment (start 154.559 98.169) (end 155.076609 98.169) (width 0.25) (layer "F.Cu") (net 9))
 (segment (start 154.559 98.169) (end 154.559 98.072) (width 0.25) (layer "F.Cu") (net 9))
 (segment (start 155.076609 98.169) (end 156.21 97.035609) (width 0.25) (layer "F.Cu") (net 9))
 (segment (start 156.972 92.331) (end 158.117 92.331) (width 0.25) (layer "F.Cu") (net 9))
 (via (at 158.496 92.71) (size 0.8) (drill 0.4) (layers "F.Cu" "B.Cu") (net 9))
 (via (at 162.052 97.917) (size 0.8) (drill 0.4) (layers "F.Cu" "B.Cu") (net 9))
 (segment (start 160.909 94.478695) (end 161.255 94.132695) (width 0.25) (layer "B.Cu") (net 9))
 (segment (start 161.925 97.4344) (end 162.052 97.917) (width 0.25) (layer "B.Cu") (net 9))
 (segment (start 159.140305 92.71) (end 158.496 92.71) (width 0.25) (layer "B.Cu") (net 9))
 (segment (start 161.255 94.132695) (end 161.255 91.405) (width 0.25) (layer "B.Cu") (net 9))
 (segment (start 160.909 96.4184) (end 160.909 94.478695) (width 0.25) (layer "B.Cu") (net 9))
 (segment (start 160.909 96.4184) (end 161.925 97.4344) (width 0.25) (layer "B.Cu") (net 9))
 (segment (start 160.909 94.478695) (end 159.140305 92.71) (width 0.25) (layer "B.Cu") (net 9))
 (segment (start 156.965 93.987595) (end 156.329405 93.987595) (width 0.25) (layer "B.Cu") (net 9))
 (segment (start 162.052 97.917) (end 161.925 97.917) (width 0.25) (layer "B.Cu") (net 9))
 (segment (start 161.255 91.405) (end 160.655 90.805) (width 0.25) (layer "B.Cu") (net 9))
 (segment (start 161.29 91.44) (end 160.655 90.805) (width 0.25) (layer "B.Cu") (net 9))
 (segment (start 157.505495 92.862495) (end 158.369 93.726) (width 0.25) (layer "B.Cu") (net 13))
 (segment (start 155.069 94.107) (end 156.313505 92.862495) (width 0.25) (layer "B.Cu") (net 13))
 (segment (start 156.313505 92.862495) (end 157.505495 92.862495) (width 0.25) (layer "B.Cu") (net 13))
 (segment (start 158.369 96.4184) (end 158.369 97.926305) (width 0.25) (layer "B.Cu") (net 13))
 (segment (start 158.369 93.726) (end 158.369 96.4184) (width 0.25) (layer "B.Cu") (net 13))
 (segment (start 155.829 98.171) (end 155.829 96.4184) (width 0.25) (layer "B.Cu") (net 13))
 (segment (start 157.399305 98.896) (end 156.554 98.896) (width 0.25) (layer "B.Cu") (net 13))
 (segment (start 158.369 97.926305) (end 157.399305 98.896) (width 0.25) (layer "B.Cu") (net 13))
 (segment (start 156.554 98.896) (end 155.829 98.171) (width 0.25) (layer "B.Cu") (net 13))
 (segment (start 151.638 99.159) (end 151.539 99.06) (width 0.25) (layer "F.Cu") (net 7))
 (segment (start 151.638 98.961) (end 151.539 99.06) (width 0.25) (layer "F.Cu") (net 7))
 (segment (start 151.638 98.044) (end 151.638 98.961) (width 0.25) (layer "F.Cu") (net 7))
 (segment (start 151.638 100.8745) (end 151.638 99.159) (width 0.25) (layer "F.Cu") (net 7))
 (via (at 151.638 98.044) (size 0.8) (drill 0.4) (layers "F.Cu" "B.Cu") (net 7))
 (segment (start 151.128 102.362) (end 151.638 101.852) (width 0.25) (layer "B.Cu") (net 7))
 (segment (start 151.638 101.852) (end 151.638 98.044) (width 0.25) (layer "B.Cu") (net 7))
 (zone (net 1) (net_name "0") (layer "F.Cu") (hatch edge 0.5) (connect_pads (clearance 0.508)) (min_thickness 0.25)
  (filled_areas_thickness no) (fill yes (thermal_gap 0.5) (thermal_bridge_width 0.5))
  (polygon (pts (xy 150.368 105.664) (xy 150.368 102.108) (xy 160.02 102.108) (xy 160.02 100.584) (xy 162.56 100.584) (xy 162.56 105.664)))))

